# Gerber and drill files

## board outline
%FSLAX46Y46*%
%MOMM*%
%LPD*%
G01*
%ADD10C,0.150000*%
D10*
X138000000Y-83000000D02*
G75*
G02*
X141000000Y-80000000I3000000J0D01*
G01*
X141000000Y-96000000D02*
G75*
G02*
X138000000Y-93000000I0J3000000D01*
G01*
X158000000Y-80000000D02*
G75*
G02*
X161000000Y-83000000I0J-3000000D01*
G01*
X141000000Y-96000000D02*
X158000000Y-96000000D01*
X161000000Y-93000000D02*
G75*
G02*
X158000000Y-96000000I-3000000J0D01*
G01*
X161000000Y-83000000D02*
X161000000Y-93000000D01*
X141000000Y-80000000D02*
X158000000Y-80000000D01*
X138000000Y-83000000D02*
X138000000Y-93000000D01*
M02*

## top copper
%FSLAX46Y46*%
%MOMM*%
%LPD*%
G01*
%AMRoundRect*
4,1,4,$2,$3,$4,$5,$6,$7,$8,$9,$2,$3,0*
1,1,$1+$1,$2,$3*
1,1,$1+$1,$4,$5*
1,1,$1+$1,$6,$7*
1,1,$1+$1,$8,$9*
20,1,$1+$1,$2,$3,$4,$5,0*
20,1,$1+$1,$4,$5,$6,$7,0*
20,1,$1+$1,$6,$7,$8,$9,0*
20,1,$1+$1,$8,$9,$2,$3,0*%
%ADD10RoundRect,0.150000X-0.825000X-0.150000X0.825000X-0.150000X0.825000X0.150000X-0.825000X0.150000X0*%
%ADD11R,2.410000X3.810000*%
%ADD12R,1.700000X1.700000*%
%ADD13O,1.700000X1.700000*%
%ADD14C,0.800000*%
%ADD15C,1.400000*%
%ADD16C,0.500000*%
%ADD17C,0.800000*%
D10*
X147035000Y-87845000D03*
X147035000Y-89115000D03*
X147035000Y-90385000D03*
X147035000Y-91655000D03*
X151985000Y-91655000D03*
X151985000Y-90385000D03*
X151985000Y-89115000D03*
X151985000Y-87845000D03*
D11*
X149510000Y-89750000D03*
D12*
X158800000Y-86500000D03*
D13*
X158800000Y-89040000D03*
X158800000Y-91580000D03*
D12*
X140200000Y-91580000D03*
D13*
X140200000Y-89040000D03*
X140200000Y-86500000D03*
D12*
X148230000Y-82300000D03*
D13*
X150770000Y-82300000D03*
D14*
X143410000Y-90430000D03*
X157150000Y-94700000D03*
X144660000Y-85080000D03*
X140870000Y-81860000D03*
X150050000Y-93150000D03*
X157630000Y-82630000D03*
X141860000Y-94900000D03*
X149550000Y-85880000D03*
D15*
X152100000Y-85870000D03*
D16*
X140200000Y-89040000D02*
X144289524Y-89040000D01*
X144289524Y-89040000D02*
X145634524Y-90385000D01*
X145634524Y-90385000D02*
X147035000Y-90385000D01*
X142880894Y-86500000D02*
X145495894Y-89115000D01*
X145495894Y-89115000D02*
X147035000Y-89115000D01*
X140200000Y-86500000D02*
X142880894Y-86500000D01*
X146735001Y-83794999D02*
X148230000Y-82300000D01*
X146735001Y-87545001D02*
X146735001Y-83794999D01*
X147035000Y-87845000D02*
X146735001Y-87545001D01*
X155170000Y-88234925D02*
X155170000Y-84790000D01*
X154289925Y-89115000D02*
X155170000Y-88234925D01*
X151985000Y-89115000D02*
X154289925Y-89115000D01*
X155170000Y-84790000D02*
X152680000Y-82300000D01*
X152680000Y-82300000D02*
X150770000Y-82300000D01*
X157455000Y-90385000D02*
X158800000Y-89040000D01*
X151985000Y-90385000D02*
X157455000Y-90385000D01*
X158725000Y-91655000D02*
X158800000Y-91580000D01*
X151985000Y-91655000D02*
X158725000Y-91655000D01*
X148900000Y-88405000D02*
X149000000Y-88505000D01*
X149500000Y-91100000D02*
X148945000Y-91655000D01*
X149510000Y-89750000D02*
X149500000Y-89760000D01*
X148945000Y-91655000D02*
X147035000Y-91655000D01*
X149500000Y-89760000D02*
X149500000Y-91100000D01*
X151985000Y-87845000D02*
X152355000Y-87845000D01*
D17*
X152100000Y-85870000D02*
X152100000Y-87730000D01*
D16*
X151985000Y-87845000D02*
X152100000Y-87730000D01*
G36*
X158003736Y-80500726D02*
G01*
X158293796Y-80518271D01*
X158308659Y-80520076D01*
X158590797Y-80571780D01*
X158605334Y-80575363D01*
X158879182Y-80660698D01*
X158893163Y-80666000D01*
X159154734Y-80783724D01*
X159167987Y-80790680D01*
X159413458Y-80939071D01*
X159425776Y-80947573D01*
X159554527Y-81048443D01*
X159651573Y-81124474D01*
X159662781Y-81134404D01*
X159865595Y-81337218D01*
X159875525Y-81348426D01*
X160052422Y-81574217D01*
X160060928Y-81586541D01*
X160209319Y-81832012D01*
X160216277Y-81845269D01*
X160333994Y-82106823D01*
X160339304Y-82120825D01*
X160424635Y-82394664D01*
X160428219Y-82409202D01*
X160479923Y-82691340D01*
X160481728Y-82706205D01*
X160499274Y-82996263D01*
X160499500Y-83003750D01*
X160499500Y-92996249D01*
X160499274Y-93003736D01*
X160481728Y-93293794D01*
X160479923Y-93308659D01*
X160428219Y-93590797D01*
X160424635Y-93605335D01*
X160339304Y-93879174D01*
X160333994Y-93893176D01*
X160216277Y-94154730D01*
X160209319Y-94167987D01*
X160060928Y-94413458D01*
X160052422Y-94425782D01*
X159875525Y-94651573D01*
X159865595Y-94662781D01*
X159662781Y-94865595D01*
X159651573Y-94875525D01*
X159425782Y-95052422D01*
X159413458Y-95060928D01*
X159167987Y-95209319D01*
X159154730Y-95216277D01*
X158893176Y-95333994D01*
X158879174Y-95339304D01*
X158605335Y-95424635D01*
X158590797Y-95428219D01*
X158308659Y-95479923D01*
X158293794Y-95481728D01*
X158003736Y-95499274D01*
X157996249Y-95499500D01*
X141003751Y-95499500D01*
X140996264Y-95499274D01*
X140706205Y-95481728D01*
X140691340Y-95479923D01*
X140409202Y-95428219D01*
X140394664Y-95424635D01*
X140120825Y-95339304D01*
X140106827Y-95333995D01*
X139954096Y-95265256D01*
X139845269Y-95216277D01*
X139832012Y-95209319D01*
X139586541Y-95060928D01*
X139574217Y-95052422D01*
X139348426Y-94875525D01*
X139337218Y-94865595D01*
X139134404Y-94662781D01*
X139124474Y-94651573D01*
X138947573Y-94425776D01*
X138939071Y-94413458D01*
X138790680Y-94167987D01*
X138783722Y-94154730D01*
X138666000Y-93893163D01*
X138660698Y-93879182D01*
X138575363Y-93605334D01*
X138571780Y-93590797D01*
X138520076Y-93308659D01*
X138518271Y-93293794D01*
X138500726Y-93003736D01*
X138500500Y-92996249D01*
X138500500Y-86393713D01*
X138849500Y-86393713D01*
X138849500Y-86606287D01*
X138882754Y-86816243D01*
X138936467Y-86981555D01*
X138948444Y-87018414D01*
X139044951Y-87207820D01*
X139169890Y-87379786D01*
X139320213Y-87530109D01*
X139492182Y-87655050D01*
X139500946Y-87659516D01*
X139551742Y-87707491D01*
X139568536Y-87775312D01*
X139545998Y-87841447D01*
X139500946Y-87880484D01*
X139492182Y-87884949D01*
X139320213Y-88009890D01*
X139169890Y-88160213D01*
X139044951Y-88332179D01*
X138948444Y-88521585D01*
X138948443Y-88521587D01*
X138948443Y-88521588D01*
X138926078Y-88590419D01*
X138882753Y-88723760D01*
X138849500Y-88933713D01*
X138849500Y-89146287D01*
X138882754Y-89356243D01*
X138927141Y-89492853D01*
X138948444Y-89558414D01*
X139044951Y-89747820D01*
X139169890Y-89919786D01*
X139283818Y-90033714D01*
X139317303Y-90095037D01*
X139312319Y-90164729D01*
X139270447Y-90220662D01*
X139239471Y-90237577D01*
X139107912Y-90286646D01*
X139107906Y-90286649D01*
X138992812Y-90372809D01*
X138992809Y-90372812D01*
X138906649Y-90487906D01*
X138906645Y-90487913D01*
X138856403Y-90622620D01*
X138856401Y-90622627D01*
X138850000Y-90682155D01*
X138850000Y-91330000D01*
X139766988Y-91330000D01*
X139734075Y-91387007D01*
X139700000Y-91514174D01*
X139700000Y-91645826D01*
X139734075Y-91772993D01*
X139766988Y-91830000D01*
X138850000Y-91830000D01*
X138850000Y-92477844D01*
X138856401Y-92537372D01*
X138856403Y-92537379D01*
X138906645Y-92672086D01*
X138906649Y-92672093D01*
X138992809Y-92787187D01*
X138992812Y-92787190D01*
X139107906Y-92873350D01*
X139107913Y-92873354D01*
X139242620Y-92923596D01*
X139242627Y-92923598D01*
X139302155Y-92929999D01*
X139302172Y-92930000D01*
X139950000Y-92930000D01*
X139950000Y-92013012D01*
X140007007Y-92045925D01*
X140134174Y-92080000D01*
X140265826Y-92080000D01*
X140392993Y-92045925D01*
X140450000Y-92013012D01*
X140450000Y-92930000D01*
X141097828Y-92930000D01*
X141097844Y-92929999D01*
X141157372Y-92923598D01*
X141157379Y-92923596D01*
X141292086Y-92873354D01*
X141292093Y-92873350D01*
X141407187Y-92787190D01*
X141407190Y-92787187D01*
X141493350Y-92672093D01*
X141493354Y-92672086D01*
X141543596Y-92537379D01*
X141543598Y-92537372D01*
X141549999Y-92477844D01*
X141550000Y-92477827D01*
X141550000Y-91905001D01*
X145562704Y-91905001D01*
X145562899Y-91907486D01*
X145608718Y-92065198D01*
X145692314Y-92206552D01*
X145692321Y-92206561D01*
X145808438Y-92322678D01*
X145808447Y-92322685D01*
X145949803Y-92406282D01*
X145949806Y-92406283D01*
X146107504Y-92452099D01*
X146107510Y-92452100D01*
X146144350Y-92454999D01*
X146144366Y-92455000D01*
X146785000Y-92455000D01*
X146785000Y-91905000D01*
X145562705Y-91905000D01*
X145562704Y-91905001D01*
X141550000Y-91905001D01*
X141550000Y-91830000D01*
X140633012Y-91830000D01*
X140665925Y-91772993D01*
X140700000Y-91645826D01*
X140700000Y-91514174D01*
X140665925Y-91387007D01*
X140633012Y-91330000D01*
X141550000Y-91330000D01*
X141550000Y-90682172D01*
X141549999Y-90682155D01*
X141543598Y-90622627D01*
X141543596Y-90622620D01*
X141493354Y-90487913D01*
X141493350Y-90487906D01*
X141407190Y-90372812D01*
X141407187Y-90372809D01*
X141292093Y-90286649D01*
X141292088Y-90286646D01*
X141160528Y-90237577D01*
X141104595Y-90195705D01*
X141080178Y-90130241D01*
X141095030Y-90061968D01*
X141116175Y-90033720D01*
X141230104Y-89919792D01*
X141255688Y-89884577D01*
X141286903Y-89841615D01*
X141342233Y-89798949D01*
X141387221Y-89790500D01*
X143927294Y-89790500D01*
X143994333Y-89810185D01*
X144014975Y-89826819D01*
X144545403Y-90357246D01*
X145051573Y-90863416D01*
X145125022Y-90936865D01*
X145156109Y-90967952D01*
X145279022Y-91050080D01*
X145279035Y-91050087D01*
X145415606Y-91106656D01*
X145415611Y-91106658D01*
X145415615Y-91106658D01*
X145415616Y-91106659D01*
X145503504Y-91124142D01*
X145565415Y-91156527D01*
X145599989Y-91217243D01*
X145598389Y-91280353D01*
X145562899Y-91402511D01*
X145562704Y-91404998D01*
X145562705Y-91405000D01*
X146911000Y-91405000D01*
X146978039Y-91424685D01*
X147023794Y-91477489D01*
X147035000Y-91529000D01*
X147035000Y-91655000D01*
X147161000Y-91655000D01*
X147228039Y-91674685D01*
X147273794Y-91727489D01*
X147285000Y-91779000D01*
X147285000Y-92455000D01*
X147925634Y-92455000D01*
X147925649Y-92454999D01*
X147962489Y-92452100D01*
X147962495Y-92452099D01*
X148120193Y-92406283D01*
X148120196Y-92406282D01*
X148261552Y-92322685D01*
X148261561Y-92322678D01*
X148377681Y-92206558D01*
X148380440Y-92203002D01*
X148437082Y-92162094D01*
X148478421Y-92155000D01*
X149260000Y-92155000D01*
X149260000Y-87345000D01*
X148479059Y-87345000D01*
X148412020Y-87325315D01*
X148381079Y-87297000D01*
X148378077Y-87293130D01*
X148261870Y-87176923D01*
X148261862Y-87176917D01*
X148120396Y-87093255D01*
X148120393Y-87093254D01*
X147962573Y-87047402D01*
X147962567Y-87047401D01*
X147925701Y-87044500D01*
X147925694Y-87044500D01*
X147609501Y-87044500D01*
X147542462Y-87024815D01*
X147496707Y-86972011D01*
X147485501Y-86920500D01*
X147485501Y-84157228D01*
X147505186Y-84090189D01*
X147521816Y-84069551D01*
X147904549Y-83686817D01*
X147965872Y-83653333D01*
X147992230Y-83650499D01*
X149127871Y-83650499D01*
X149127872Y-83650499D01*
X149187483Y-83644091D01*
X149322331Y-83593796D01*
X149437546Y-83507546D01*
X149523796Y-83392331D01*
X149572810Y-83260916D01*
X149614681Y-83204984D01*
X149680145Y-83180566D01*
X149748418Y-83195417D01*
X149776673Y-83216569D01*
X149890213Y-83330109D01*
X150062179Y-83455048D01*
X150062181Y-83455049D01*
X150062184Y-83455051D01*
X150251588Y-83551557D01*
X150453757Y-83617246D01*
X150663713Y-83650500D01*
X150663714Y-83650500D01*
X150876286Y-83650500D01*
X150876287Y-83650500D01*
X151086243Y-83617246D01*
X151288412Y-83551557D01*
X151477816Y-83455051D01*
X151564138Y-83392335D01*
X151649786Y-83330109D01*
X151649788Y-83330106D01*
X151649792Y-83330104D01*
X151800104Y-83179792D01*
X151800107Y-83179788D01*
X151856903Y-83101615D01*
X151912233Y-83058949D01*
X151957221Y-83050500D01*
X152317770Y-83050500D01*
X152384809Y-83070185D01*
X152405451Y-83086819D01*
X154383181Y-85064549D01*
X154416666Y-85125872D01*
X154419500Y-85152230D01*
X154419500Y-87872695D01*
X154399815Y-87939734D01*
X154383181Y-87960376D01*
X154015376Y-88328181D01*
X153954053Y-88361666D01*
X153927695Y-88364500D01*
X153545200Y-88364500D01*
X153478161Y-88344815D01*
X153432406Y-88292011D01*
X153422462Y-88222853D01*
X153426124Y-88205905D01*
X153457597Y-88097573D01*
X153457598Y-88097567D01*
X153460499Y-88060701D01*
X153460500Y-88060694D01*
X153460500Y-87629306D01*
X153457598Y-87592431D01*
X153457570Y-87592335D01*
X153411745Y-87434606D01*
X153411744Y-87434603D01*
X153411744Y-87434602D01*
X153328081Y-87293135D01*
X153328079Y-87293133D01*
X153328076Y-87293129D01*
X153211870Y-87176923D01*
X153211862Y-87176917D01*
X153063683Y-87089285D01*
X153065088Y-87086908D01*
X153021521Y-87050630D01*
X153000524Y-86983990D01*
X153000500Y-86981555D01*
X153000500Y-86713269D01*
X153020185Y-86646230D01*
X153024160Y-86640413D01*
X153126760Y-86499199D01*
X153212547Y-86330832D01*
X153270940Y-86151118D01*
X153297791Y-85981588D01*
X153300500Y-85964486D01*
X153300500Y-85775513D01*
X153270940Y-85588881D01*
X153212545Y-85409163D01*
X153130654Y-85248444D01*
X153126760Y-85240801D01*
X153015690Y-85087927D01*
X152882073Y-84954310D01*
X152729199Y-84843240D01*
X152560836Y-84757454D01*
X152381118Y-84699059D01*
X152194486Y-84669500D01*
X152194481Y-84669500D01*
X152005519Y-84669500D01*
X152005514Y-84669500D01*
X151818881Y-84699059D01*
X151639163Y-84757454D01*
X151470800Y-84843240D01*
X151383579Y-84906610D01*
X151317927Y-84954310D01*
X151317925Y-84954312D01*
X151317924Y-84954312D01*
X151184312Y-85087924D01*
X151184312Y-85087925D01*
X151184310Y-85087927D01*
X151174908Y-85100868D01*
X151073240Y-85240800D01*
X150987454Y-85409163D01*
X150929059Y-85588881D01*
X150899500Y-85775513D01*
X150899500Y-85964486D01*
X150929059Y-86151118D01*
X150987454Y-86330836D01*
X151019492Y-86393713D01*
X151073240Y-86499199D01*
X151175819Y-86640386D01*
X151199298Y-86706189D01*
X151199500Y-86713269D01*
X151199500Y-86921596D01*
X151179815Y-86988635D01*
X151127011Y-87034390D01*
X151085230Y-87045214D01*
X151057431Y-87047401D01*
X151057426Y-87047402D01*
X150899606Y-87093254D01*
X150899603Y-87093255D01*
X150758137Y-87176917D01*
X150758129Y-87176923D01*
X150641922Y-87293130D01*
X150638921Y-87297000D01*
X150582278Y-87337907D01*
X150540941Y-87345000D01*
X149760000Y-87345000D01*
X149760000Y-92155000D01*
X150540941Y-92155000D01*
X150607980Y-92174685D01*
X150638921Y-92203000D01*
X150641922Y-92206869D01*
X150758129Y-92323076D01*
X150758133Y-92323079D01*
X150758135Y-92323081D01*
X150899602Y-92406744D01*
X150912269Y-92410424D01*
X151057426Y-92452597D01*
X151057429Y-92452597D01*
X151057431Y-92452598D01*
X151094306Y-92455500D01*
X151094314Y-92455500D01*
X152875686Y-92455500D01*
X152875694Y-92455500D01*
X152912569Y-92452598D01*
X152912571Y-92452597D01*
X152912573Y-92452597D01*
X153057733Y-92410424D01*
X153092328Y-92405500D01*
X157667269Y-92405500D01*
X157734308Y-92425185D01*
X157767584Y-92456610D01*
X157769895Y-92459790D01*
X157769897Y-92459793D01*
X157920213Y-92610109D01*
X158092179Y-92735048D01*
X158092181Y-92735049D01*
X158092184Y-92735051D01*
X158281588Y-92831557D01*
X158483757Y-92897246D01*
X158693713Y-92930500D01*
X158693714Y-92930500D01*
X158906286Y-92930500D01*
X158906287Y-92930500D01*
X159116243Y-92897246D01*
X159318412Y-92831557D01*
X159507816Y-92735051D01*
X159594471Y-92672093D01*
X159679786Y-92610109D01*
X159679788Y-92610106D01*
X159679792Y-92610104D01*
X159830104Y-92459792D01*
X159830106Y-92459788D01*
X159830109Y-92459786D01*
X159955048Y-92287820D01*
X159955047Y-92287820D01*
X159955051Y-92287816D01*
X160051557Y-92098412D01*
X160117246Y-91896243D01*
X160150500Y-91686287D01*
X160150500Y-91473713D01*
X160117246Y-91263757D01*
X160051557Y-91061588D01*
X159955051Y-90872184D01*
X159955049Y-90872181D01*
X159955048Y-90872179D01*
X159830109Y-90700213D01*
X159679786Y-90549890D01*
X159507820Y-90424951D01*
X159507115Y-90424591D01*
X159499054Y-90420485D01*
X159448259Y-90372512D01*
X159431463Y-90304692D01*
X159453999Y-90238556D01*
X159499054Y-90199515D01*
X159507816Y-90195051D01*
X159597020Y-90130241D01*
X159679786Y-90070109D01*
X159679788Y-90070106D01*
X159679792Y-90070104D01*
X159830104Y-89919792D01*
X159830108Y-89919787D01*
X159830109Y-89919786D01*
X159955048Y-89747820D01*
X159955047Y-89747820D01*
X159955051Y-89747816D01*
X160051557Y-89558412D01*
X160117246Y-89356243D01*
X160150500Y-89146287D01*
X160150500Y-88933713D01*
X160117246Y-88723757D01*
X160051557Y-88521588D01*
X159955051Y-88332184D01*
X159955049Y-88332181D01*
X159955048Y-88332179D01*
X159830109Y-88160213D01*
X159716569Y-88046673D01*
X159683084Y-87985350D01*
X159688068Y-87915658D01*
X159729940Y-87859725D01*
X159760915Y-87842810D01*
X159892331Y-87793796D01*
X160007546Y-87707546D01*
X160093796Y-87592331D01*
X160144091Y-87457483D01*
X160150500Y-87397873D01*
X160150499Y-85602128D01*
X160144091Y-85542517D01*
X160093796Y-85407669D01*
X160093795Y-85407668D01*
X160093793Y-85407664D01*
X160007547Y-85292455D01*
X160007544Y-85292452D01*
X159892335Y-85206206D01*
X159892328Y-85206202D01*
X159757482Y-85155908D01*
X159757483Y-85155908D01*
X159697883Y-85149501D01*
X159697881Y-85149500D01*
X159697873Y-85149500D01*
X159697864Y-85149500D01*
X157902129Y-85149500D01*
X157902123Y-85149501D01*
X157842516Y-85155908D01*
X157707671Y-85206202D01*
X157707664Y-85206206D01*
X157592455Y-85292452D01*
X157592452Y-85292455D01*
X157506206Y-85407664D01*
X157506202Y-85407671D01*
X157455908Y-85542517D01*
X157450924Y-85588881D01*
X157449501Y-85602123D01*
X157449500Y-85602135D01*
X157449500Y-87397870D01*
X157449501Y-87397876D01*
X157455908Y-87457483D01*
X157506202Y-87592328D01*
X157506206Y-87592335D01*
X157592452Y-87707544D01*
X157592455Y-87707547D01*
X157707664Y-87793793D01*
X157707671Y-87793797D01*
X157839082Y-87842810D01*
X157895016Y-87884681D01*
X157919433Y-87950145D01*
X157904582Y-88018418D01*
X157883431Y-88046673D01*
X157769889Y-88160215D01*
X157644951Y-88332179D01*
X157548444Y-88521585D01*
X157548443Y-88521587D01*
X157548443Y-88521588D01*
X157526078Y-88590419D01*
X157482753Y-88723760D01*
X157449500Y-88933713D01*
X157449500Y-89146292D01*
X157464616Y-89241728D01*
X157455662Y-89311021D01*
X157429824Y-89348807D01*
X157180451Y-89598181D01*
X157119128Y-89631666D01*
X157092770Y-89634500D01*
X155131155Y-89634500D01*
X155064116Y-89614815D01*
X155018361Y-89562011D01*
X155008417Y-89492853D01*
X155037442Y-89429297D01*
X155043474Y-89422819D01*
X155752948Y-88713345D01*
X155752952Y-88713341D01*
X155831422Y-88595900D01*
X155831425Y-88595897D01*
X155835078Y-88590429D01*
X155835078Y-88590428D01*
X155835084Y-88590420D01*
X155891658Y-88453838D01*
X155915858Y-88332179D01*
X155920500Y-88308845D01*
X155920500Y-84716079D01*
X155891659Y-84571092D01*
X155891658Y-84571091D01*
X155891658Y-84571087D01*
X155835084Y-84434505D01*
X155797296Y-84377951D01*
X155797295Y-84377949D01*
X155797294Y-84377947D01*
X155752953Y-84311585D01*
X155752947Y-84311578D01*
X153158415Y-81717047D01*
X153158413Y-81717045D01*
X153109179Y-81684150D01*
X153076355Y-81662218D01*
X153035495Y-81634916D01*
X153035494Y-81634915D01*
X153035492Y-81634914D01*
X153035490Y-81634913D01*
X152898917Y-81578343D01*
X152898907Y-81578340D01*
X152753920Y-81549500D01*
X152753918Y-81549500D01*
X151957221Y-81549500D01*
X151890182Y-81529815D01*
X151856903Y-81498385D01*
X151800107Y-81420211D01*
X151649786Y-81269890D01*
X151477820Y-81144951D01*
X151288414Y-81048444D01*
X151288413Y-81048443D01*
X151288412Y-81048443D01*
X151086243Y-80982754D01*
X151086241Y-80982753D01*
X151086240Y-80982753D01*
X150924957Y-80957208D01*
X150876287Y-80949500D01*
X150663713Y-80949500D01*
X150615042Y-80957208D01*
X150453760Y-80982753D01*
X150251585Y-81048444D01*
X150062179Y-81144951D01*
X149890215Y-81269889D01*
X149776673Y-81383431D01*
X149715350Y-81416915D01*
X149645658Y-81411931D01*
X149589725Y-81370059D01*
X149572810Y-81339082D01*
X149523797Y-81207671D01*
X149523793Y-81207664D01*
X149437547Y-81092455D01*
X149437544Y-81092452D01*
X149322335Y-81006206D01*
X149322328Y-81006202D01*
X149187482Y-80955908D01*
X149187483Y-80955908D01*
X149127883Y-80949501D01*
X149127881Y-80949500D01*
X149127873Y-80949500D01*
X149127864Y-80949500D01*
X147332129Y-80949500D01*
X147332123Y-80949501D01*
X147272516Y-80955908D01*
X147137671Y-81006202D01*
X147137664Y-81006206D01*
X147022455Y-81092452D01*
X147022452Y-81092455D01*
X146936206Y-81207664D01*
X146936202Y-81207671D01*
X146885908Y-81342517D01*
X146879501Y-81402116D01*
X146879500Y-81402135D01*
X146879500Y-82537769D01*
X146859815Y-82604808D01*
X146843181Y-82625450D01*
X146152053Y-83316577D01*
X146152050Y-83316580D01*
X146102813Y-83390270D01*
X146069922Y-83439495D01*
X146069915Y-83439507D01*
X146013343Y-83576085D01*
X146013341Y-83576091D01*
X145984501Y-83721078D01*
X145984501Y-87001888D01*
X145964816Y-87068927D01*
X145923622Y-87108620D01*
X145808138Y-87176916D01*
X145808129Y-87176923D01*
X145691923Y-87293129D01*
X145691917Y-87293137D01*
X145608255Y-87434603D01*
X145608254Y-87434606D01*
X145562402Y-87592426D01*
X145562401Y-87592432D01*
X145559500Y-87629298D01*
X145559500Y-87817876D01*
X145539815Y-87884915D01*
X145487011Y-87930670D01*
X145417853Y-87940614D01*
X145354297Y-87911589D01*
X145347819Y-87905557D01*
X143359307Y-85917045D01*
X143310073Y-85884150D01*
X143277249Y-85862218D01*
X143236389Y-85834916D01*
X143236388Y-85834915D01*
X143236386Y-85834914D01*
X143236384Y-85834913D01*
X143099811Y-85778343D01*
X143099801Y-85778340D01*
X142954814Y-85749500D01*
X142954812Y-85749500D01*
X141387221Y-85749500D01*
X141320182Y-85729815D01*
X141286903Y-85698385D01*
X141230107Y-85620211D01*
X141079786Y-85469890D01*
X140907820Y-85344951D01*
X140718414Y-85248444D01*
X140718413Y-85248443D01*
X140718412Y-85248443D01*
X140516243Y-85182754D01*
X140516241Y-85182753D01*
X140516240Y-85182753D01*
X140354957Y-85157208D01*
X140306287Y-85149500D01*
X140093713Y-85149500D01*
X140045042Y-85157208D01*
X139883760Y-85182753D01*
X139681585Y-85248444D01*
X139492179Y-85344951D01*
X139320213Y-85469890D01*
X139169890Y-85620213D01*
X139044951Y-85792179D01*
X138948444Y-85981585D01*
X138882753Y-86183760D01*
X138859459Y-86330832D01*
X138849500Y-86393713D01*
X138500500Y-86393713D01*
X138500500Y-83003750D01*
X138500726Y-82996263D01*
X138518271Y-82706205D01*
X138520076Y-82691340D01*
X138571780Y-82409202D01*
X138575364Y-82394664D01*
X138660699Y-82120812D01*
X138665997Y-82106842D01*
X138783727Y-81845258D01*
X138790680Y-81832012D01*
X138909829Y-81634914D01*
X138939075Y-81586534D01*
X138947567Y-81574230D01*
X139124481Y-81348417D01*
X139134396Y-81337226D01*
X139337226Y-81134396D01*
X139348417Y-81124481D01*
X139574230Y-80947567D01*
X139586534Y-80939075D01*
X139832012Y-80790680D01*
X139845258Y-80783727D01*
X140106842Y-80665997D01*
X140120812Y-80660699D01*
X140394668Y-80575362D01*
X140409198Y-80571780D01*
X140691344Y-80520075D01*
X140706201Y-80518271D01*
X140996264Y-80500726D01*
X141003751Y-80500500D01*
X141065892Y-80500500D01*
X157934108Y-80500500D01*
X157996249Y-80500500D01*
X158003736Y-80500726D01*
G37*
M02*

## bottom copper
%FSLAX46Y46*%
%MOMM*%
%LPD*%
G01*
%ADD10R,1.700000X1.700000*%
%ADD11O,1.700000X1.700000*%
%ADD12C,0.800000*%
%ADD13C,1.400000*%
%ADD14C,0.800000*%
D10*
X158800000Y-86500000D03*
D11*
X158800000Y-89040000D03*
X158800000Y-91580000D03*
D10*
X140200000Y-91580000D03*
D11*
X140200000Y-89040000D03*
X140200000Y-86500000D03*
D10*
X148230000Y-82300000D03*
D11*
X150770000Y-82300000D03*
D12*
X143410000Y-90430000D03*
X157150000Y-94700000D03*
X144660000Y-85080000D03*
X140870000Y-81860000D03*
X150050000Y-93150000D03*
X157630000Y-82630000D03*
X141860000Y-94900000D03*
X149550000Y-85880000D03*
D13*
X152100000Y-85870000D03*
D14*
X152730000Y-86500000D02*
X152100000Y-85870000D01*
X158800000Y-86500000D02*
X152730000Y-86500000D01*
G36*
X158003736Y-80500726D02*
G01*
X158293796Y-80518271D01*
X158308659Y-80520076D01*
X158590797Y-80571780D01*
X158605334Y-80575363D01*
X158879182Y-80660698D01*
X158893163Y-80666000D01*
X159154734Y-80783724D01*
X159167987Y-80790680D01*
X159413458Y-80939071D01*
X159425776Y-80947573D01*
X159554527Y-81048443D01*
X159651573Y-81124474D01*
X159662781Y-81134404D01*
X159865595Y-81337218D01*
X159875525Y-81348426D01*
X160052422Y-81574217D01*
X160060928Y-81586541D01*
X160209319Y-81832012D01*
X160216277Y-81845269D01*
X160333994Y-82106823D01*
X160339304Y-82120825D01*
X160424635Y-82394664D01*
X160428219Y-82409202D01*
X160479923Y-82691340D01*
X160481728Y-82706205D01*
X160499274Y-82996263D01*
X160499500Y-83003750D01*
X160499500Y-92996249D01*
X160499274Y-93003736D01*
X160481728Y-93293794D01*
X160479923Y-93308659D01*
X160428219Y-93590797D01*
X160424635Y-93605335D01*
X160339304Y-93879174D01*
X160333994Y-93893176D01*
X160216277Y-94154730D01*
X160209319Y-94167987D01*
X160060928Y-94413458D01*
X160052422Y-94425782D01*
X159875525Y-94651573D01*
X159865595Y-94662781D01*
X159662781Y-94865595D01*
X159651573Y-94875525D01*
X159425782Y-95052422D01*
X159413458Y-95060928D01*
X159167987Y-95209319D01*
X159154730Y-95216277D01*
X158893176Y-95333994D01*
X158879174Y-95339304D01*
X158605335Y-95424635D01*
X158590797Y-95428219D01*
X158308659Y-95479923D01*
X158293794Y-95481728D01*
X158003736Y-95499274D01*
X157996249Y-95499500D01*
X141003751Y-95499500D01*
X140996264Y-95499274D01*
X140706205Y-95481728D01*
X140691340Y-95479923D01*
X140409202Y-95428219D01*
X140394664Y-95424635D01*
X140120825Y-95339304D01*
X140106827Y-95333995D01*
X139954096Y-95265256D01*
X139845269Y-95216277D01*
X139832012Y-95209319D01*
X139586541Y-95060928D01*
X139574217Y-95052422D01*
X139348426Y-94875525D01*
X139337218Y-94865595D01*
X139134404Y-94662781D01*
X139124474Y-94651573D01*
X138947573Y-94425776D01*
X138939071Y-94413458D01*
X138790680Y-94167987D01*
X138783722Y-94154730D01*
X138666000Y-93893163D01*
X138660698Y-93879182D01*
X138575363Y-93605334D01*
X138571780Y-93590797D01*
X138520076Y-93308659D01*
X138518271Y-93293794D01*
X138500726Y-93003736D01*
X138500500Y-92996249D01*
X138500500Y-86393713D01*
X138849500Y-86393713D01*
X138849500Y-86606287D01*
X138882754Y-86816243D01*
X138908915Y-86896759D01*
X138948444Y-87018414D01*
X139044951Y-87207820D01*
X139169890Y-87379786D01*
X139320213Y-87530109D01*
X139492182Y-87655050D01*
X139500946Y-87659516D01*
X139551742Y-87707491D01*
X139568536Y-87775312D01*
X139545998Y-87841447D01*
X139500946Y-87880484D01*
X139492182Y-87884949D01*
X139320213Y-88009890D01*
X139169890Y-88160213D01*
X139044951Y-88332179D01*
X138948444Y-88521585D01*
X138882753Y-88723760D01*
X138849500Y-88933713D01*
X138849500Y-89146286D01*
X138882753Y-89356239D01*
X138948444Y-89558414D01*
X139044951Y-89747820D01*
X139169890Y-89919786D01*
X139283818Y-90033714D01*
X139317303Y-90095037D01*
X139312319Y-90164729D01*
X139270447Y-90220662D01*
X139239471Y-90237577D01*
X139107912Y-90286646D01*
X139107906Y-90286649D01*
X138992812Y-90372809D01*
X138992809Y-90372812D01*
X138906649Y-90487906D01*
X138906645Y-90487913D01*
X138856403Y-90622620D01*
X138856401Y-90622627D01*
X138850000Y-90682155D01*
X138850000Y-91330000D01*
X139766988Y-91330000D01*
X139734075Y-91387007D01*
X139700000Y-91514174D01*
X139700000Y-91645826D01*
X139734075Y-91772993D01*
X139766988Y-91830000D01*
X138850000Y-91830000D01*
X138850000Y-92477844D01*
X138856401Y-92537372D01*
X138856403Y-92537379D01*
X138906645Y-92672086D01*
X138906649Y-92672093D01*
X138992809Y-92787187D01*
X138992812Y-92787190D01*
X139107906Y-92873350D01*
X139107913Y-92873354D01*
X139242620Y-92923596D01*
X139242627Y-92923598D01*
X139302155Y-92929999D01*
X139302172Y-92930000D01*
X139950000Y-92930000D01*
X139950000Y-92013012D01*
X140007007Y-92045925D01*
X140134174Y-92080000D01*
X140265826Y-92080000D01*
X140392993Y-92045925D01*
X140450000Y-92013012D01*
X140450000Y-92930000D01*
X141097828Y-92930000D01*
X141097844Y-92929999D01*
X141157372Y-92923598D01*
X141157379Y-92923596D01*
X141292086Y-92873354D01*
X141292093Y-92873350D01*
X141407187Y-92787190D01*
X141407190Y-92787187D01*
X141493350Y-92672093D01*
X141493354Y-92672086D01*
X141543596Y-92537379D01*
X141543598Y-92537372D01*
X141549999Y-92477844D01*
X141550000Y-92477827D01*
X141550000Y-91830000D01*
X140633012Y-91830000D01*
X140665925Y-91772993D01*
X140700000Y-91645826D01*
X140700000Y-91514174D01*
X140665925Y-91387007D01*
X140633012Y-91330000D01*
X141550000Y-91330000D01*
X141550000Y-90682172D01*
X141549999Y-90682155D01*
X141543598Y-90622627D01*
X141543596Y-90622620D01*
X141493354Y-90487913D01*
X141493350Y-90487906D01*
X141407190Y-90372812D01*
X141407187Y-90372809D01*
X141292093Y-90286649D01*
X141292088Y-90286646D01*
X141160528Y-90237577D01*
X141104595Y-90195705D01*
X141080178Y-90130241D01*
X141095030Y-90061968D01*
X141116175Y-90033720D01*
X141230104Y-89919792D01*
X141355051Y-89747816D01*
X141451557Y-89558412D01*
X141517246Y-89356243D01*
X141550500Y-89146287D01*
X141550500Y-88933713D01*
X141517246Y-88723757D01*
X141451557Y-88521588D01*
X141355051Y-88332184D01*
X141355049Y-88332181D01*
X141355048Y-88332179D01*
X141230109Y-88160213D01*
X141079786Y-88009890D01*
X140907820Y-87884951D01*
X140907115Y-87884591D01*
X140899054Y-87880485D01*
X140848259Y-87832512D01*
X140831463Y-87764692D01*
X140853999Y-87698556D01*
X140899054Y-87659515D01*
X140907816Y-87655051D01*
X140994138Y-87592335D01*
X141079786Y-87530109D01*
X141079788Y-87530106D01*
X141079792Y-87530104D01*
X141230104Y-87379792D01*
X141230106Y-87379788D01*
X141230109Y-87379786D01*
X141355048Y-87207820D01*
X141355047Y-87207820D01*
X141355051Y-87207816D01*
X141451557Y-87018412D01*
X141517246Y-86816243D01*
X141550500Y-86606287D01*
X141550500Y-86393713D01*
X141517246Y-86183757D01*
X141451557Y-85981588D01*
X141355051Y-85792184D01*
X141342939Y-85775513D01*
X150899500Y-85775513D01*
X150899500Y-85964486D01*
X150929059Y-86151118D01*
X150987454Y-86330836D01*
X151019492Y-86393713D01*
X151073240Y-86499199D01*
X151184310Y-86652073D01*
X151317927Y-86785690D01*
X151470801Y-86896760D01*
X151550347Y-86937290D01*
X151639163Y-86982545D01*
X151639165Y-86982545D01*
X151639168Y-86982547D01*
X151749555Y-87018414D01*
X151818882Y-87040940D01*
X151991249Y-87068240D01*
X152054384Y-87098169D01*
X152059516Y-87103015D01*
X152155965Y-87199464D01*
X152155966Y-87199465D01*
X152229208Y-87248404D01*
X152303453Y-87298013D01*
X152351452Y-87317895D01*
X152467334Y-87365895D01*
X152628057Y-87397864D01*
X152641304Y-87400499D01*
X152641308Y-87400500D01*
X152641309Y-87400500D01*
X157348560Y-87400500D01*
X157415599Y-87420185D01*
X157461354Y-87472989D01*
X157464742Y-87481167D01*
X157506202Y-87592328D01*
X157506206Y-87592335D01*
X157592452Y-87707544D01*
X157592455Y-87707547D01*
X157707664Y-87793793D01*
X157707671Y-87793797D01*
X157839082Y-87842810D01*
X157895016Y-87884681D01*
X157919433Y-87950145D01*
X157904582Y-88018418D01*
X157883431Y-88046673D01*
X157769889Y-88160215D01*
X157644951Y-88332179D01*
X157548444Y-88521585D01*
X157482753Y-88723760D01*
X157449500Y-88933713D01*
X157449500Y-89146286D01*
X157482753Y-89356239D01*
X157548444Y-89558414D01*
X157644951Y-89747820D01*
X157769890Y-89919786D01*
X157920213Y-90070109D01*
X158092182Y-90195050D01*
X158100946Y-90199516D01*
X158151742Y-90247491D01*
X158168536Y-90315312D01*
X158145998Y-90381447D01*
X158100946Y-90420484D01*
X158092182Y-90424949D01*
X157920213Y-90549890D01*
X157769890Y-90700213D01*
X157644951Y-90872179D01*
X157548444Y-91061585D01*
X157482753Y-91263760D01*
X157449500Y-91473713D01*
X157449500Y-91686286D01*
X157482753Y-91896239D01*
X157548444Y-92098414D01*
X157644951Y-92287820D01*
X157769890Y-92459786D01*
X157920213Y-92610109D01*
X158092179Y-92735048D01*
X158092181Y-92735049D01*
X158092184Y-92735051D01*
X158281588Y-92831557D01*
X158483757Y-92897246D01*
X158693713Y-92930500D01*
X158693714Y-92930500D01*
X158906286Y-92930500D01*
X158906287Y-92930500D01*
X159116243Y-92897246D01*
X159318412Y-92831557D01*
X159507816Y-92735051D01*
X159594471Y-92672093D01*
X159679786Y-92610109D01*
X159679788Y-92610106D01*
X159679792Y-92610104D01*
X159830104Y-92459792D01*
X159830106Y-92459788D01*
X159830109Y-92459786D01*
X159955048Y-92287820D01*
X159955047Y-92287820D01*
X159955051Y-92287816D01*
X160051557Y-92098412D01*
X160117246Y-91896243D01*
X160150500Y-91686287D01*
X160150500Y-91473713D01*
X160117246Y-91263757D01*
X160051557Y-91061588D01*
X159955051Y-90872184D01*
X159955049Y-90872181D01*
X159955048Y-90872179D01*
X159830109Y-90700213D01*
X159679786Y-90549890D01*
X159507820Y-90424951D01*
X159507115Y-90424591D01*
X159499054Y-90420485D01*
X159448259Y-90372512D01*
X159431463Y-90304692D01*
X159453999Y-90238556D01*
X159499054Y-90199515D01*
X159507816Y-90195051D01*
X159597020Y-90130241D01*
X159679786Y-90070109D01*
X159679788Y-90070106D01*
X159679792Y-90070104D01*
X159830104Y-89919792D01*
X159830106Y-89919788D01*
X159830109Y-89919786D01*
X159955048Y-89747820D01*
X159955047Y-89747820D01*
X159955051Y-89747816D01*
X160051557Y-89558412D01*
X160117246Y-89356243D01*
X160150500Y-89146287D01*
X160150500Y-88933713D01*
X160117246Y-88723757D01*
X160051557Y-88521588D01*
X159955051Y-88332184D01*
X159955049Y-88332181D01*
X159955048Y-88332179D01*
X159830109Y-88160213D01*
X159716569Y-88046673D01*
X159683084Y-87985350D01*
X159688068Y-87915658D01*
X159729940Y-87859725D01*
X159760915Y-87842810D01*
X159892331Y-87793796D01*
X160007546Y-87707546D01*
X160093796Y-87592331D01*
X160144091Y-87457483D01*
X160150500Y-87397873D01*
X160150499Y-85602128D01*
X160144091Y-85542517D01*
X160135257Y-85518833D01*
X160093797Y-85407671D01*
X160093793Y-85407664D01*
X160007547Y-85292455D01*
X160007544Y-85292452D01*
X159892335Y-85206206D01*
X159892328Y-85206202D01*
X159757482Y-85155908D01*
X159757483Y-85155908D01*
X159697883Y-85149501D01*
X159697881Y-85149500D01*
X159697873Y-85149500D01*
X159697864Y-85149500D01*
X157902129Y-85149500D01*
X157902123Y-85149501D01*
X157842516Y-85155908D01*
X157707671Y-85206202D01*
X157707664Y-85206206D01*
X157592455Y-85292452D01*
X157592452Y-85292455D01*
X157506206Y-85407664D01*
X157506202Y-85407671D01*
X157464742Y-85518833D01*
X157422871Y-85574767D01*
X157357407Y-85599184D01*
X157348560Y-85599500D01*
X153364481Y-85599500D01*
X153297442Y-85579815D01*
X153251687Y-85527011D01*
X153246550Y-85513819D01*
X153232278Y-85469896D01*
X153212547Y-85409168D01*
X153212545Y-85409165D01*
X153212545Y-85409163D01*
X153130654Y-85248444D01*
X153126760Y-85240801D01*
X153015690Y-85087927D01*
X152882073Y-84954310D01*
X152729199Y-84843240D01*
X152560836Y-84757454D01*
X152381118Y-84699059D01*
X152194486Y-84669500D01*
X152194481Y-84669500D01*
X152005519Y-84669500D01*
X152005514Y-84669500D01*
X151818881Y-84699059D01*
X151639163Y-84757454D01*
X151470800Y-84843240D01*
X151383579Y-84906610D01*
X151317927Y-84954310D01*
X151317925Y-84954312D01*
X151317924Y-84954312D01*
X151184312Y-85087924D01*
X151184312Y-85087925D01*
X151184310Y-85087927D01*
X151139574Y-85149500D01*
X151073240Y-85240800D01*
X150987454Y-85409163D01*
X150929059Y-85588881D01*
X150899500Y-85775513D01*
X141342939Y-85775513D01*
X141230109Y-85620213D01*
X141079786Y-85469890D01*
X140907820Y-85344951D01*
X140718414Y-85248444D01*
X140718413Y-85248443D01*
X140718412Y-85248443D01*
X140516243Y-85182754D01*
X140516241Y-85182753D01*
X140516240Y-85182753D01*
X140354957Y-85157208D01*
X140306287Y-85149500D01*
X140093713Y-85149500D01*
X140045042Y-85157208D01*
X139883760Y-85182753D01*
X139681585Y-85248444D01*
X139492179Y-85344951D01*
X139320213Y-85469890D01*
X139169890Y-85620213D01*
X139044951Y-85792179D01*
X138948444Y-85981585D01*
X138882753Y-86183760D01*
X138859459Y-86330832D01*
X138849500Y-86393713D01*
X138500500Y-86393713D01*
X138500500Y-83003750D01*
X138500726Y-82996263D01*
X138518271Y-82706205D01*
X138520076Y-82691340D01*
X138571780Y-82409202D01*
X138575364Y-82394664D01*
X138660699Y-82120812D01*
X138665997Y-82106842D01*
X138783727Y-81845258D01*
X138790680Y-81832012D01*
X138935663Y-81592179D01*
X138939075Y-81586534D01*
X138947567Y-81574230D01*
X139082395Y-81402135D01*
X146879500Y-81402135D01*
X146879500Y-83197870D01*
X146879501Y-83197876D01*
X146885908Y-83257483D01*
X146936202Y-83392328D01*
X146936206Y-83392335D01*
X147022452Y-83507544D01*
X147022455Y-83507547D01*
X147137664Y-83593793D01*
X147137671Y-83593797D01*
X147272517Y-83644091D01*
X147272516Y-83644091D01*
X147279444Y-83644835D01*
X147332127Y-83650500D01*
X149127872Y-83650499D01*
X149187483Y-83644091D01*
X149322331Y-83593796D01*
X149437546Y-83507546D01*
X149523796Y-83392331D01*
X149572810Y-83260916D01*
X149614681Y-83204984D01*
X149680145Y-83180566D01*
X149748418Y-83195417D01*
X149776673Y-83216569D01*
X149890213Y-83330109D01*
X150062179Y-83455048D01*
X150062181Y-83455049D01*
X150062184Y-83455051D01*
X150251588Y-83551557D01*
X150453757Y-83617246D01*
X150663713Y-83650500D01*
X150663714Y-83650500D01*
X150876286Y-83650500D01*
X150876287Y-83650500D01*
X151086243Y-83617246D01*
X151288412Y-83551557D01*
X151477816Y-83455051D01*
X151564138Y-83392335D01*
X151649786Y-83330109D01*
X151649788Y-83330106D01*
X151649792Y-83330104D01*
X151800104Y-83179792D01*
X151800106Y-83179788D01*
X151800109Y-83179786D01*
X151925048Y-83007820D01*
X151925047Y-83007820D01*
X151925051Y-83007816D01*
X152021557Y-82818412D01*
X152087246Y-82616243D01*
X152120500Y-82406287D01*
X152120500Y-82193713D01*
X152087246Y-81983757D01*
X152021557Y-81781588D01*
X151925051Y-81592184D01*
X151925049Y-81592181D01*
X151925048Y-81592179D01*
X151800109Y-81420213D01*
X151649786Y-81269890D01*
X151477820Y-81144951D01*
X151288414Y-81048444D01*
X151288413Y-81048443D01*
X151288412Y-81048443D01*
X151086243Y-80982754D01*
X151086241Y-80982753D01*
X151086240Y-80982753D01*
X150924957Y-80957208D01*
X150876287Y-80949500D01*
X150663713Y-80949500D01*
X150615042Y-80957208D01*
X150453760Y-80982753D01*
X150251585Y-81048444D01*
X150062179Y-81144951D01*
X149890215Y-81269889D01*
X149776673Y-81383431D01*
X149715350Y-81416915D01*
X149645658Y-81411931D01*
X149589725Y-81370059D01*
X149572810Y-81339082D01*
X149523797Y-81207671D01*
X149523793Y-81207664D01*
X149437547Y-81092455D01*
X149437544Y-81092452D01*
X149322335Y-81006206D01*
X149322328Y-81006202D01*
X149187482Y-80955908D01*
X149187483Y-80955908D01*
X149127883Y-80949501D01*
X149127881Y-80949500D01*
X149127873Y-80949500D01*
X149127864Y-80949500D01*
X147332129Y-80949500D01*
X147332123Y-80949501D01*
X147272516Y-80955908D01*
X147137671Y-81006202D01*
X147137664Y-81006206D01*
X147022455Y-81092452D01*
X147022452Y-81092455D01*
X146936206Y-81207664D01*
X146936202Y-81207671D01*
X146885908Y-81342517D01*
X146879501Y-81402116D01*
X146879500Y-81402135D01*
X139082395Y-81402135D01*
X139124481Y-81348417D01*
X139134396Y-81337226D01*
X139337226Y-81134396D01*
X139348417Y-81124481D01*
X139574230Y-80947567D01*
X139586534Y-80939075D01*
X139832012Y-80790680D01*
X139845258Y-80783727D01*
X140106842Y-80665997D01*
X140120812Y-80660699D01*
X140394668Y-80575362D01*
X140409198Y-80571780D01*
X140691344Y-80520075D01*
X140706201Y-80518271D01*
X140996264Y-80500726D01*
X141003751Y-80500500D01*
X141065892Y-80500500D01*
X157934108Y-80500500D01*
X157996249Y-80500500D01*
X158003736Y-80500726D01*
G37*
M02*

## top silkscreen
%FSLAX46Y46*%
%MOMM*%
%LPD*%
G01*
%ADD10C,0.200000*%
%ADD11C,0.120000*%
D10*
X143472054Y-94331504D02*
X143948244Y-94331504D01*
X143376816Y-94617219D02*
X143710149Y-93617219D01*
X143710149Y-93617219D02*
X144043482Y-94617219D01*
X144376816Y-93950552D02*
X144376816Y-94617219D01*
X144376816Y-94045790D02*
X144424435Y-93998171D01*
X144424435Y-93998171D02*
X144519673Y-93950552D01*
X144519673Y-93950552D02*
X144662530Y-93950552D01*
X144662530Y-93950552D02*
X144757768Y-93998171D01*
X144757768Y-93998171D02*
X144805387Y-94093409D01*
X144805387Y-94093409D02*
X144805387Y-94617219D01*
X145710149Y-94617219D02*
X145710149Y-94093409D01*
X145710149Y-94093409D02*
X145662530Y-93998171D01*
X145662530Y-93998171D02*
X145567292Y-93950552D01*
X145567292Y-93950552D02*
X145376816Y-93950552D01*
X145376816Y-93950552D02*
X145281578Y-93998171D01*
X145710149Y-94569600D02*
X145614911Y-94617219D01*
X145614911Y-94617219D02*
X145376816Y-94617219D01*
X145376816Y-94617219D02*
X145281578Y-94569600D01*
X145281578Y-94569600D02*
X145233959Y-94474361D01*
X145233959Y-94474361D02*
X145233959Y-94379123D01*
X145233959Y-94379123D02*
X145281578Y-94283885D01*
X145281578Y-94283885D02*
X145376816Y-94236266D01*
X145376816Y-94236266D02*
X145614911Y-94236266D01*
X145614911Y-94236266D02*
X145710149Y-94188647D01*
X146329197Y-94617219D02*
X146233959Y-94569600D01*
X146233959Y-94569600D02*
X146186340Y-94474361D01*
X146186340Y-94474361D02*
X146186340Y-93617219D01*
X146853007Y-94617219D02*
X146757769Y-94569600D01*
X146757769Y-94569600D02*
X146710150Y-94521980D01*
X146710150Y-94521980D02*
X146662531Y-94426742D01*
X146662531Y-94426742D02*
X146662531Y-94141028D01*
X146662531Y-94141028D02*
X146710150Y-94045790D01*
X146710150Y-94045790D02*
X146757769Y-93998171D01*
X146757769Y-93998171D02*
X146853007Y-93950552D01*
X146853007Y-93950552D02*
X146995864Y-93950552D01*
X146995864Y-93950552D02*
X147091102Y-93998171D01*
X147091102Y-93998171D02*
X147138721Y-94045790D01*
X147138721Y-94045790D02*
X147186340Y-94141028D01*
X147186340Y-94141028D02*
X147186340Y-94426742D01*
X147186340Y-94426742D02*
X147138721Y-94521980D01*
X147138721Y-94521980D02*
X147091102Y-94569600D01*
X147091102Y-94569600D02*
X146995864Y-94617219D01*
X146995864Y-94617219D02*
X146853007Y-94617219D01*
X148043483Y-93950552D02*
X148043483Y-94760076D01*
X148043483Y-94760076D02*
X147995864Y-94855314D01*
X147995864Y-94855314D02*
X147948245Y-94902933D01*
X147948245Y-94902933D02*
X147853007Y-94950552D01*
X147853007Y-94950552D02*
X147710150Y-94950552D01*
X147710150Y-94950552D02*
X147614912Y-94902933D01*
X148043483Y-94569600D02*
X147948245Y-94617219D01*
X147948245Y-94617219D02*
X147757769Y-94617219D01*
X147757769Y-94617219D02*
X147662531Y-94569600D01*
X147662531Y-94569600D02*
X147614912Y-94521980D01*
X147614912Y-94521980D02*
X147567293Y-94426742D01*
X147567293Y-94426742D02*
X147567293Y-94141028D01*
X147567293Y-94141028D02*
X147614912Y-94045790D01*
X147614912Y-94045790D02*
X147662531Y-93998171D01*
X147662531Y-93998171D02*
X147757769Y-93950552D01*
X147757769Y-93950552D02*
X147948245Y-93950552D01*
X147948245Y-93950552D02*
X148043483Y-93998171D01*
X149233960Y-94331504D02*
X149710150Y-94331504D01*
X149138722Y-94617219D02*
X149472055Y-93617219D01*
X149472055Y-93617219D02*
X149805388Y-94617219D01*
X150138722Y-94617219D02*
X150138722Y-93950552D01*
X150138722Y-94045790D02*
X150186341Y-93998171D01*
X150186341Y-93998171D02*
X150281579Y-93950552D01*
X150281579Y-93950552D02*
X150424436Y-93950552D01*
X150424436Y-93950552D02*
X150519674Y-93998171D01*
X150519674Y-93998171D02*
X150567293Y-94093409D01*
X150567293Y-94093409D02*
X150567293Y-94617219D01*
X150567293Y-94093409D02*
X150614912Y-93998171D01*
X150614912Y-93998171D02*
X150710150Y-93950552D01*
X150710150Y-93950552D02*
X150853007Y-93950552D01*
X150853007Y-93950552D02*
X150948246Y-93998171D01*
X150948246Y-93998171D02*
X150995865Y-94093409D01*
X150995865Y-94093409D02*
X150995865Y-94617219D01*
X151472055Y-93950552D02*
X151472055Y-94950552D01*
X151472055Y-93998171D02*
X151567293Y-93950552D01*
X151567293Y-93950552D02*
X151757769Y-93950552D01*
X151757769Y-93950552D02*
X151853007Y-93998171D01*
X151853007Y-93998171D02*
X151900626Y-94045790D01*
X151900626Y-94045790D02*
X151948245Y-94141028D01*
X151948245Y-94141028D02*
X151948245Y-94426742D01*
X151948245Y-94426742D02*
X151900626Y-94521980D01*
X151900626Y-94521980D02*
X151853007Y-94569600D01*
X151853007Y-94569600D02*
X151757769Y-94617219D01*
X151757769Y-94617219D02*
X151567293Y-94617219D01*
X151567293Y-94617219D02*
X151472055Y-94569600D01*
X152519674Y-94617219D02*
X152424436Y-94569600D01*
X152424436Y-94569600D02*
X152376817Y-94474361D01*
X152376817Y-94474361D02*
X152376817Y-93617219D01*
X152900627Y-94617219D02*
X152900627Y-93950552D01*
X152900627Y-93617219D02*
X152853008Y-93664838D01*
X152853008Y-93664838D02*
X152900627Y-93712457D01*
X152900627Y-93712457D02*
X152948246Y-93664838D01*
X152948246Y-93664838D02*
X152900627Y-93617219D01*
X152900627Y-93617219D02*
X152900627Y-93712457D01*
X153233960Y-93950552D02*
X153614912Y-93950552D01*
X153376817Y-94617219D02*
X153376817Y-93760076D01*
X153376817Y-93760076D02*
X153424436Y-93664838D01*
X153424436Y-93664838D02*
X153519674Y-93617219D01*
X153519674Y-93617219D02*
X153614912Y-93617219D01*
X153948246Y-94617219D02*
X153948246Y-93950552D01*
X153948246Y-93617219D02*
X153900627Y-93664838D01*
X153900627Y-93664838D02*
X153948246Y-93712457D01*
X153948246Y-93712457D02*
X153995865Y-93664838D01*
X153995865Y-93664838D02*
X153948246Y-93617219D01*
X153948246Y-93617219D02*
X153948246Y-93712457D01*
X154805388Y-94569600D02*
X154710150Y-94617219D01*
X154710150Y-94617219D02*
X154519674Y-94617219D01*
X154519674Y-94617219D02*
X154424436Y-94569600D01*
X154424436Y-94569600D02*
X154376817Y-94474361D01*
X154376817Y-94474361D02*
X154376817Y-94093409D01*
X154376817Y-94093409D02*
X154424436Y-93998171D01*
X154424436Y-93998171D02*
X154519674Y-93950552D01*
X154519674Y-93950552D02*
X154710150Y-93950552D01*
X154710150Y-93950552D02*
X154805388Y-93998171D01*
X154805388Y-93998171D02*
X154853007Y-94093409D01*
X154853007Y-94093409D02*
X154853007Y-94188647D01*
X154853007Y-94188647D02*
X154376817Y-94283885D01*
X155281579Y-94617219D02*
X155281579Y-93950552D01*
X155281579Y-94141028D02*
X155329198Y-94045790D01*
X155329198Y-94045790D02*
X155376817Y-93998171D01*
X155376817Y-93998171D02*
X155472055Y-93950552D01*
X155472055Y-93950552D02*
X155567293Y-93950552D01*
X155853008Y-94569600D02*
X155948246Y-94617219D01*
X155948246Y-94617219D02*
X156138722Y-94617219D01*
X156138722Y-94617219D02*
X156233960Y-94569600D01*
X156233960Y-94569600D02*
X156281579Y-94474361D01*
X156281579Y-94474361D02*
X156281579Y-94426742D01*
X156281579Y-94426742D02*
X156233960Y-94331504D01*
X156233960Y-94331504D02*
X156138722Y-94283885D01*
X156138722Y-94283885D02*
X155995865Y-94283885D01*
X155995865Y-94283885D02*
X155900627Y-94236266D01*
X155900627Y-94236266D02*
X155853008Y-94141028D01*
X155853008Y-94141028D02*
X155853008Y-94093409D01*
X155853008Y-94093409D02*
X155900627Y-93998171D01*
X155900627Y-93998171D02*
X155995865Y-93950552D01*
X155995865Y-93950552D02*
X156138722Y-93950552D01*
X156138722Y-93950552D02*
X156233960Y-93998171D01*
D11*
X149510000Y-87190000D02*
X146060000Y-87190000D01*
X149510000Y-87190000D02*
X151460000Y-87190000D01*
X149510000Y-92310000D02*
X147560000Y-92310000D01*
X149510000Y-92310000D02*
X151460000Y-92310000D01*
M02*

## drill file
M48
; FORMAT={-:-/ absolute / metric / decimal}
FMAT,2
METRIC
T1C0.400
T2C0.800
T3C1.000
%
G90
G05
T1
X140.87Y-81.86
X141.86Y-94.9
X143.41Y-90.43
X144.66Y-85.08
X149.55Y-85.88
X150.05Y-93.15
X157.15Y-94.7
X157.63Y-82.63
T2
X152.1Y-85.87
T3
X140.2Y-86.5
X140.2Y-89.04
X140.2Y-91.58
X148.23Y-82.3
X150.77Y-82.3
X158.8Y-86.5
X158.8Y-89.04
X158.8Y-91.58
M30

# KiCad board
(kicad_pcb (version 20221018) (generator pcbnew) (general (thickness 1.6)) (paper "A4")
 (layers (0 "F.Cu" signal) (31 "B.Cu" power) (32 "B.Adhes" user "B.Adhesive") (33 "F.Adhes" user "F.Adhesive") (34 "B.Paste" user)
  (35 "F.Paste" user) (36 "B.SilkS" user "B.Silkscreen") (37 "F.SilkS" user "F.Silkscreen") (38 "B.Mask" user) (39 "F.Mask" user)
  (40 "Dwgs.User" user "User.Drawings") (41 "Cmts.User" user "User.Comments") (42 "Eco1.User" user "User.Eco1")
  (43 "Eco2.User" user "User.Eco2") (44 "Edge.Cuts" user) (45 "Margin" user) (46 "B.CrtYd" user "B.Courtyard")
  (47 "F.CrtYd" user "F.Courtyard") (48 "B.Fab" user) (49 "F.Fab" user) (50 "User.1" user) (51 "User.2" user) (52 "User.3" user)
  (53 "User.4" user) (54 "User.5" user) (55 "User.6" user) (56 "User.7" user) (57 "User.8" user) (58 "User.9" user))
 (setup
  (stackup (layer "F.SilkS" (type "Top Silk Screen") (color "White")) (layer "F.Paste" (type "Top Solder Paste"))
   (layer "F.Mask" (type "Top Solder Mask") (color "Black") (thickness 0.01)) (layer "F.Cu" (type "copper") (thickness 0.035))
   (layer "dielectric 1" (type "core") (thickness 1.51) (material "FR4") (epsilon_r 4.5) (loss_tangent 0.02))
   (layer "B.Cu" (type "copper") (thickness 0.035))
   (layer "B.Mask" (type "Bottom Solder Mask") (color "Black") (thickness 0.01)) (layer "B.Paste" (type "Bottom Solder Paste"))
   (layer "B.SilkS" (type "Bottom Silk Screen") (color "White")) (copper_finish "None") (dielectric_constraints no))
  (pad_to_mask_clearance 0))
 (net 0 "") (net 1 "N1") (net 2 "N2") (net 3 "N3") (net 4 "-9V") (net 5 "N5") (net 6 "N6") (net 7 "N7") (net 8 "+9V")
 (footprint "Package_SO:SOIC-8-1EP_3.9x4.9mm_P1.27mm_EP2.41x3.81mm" (layer "F.Cu") (at 149.51 89.75)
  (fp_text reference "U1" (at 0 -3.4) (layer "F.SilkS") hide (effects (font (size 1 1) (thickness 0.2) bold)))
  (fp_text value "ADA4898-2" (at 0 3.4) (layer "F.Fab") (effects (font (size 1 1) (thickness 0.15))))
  (fp_line (start 0 -2.56) (end -3.45 -2.56) (stroke (width 0.12) (type solid)) (layer "F.SilkS"))
  (fp_line (start 0 -2.56) (end 1.95 -2.56) (stroke (width 0.12) (type solid)) (layer "F.SilkS"))
  (fp_line (start 0 2.56) (end -1.95 2.56) (stroke (width 0.12) (type solid)) (layer "F.SilkS"))
  (fp_line (start 0 2.56) (end 1.95 2.56) (stroke (width 0.12) (type solid)) (layer "F.SilkS"))
  (pad "" smd roundrect (at -0.6 -0.95) (size 0.97 1.54) (layers "F.Paste") (roundrect_rratio 0.25))
  (pad "" smd roundrect (at -0.6 0.95) (size 0.97 1.54) (layers "F.Paste") (roundrect_rratio 0.25))
  (pad "" smd roundrect (at 0.6 -0.95) (size 0.97 1.54) (layers "F.Paste") (roundrect_rratio 0.25))
  (pad "" smd roundrect (at 0.6 0.95) (size 0.97 1.54) (layers "F.Paste") (roundrect_rratio 0.25))
  (pad "1" smd roundrect (at -2.475 -1.905) (size 1.95 0.6) (layers "F.Cu" "F.Paste" "F.Mask") (roundrect_rratio 0.25) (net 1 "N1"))
  (pad "2" smd roundrect (at -2.475 -0.635) (size 1.95 0.6) (layers "F.Cu" "F.Paste" "F.Mask") (roundrect_rratio 0.25) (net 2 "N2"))
  (pad "3" smd roundrect (at -2.475 0.635) (size 1.95 0.6) (layers "F.Cu" "F.Paste" "F.Mask") (roundrect_rratio 0.25) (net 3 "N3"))
  (pad "4" smd roundrect (at -2.475 1.905) (size 1.95 0.6) (layers "F.Cu" "F.Paste" "F.Mask") (roundrect_rratio 0.25) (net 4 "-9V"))
  (pad "5" smd roundrect (at 2.475 1.905) (size 1.95 0.6) (layers "F.Cu" "F.Paste" "F.Mask") (roundrect_rratio 0.25) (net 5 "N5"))
  (pad "6" smd roundrect (at 2.475 0.635) (size 1.95 0.6) (layers "F.Cu" "F.Paste" "F.Mask") (roundrect_rratio 0.25) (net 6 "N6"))
  (pad "7" smd roundrect (at 2.475 -0.635) (size 1.95 0.6) (layers "F.Cu" "F.Paste" "F.Mask") (roundrect_rratio 0.25) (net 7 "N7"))
  (pad "8" smd roundrect (at 2.475 -1.905) (size 1.95 0.6) (layers "F.Cu" "F.Paste" "F.Mask") (roundrect_rratio 0.25) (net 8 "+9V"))
  (pad "9" smd rect (at 0 0) (size 2.41 3.81) (layers "F.Cu" "F.Mask") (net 4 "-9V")))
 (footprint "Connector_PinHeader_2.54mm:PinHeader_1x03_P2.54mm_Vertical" (layer "B.Cu") (at 158.8 86.5 180)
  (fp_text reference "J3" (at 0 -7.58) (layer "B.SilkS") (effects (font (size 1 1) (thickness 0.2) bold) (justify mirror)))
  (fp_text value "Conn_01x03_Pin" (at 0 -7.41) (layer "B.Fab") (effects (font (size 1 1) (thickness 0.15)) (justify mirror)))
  (pad "1" thru_hole rect (at 0 0 180) (size 1.7 1.7) (drill 1) (layers "*.Cu" "*.Mask") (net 8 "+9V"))
  (pad "2" thru_hole oval (at 0 -2.54 180) (size 1.7 1.7) (drill 1) (layers "*.Cu" "*.Mask") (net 6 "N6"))
  (pad "3" thru_hole oval (at 0 -5.08 180) (size 1.7 1.7) (drill 1) (layers "*.Cu" "*.Mask") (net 5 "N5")))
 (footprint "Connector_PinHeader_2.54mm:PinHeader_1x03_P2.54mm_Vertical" (layer "B.Cu") (at 140.2 91.58)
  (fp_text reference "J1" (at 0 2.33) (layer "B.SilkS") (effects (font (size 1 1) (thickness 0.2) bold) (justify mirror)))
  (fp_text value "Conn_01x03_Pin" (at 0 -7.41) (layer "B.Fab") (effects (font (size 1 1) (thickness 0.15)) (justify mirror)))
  (pad "1" thru_hole rect (at 0 0) (size 1.7 1.7) (drill 1) (layers "*.Cu" "*.Mask") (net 4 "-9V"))
  (pad "2" thru_hole oval (at 0 -2.54) (size 1.7 1.7) (drill 1) (layers "*.Cu" "*.Mask") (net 3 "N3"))
  (pad "3" thru_hole oval (at 0 -5.08) (size 1.7 1.7) (drill 1) (layers "*.Cu" "*.Mask") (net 2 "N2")))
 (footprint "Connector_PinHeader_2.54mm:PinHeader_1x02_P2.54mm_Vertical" (layer "B.Cu") (at 148.23 82.3 -90)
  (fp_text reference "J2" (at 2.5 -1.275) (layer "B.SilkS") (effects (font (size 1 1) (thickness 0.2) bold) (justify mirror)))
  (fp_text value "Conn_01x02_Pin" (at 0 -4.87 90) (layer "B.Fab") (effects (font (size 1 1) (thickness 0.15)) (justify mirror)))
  (pad "1" thru_hole rect (at 0 0 270) (size 1.7 1.7) (drill 1) (layers "*.Cu" "*.Mask") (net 1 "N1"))
  (pad "2" thru_hole oval (at 0 -2.54 270) (size 1.7 1.7) (drill 1) (layers "*.Cu" "*.Mask") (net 7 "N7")))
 (gr_arc (start 138 83) (mid 138.87868 80.87868) (end 141 80) (stroke (width 0.15) (type default)) (layer "Edge.Cuts"))
 (gr_arc (start 141 96) (mid 138.87868 95.12132) (end 138 93) (stroke (width 0.15) (type default)) (layer "Edge.Cuts"))
 (gr_arc (start 158 80) (mid 160.12132 80.87868) (end 161 83) (stroke (width 0.15) (type default)) (layer "Edge.Cuts"))
 (gr_line (start 141 96) (end 158 96) (stroke (width 0.15) (type default)) (layer "Edge.Cuts"))
 (gr_arc (start 161 93) (mid 160.12132 95.12132) (end 158 96) (stroke (width 0.15) (type default)) (layer "Edge.Cuts"))
 (gr_line (start 161 83) (end 161 93) (stroke (width 0.15) (type default)) (layer "Edge.Cuts"))
 (gr_line (start 141 80) (end 158 80) (stroke (width 0.15) (type default)) (layer "Edge.Cuts"))
 (gr_line (start 138 83) (end 138 93) (stroke (width 0.15) (type default)) (layer "Edge.Cuts"))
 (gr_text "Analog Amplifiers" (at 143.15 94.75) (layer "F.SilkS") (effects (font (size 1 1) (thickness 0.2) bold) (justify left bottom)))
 (segment (start 140.2 89.04) (end 144.289524 89.04) (width 0.5) (layer "F.Cu") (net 3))
 (segment (start 144.289524 89.04) (end 145.634524 90.385) (width 0.5) (layer "F.Cu") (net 3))
 (segment (start 145.634524 90.385) (end 147.035 90.385) (width 0.5) (layer "F.Cu") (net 3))
 (segment (start 142.880894 86.5) (end 145.495894 89.115) (width 0.5) (layer "F.Cu") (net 2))
 (segment (start 145.495894 89.115) (end 147.035 89.115) (width 0.5) (layer "F.Cu") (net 2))
 (segment (start 140.2 86.5) (end 142.880894 86.5) (width 0.5) (layer "F.Cu") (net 2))
 (segment (start 146.735001 83.794999) (end 148.23 82.3) (width 0.5) (layer "F.Cu") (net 1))
 (segment (start 146.735001 87.545001) (end 146.735001 83.794999) (width 0.5) (layer "F.Cu") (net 1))
 (segment (start 147.035 87.845) (end 146.735001 87.545001) (width 0.5) (layer "F.Cu") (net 1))
 (segment (start 155.17 88.234925) (end 155.17 84.79) (width 0.5) (layer "F.Cu") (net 7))
 (segment (start 154.289925 89.115) (end 155.17 88.234925) (width 0.5) (layer "F.Cu") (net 7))
 (segment (start 151.985 89.115) (end 154.289925 89.115) (width 0.5) (layer "F.Cu") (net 7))
 (segment (start 155.17 84.79) (end 152.68 82.3) (width 0.5) (layer "F.Cu") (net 7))
 (segment (start 152.68 82.3) (end 150.77 82.3) (width 0.5) (layer "F.Cu") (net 7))
 (segment (start 157.455 90.385) (end 158.8 89.04) (width 0.5) (layer "F.Cu") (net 6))
 (segment (start 151.985 90.385) (end 157.455 90.385) (width 0.5) (layer "F.Cu") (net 6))
 (segment (start 158.725 91.655) (end 158.8 91.58) (width 0.5) (layer "F.Cu") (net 5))
 (segment (start 151.985 91.655) (end 158.725 91.655) (width 0.5) (layer "F.Cu") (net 5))
 (segment (start 148.9 88.405) (end 149 88.505) (width 0.5) (layer "F.Cu") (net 4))
 (segment (start 149.5 91.1) (end 148.945 91.655) (width 0.5) (layer "F.Cu") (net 4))
 (segment (start 149.51 89.75) (end 149.5 89.76) (width 0.5) (layer "F.Cu") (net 4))
 (segment (start 148.945 91.655) (end 147.035 91.655) (width 0.5) (layer "F.Cu") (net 4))
 (segment (start 149.5 89.76) (end 149.5 91.1) (width 0.5) (layer "F.Cu") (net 4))
 (via (at 143.41 90.43) (size 0.8) (drill 0.4) (layers "F.Cu" "B.Cu") (free) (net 4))
 (via (at 157.15 94.7) (size 0.8) (drill 0.4) (layers "F.Cu" "B.Cu") (free) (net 4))
 (via (at 144.66 85.08) (size 0.8) (drill 0.4) (layers "F.Cu" "B.Cu") (free) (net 4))
 (via (at 140.87 81.86) (size 0.8) (drill 0.4) (layers "F.Cu" "B.Cu") (free) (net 4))
 (via (at 150.05 93.15) (size 0.8) (drill 0.4) (layers "F.Cu" "B.Cu") (free) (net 4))
 (via (at 157.63 82.63) (size 0.8) (drill 0.4) (layers "F.Cu" "B.Cu") (free) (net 4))
 (via (at 141.86 94.9) (size 0.8) (drill 0.4) (layers "F.Cu" "B.Cu") (free) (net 4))
 (via (at 149.55 85.88) (size 0.8) (drill 0.4) (layers "F.Cu" "B.Cu") (free) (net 4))
 (segment (start 151.985 87.845) (end 152.355 87.845) (width 0.5) (layer "F.Cu") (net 8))
 (segment (start 152.1 85.87) (end 152.1 87.73) (width 0.8) (layer "F.Cu") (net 8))
 (segment (start 151.985 87.845) (end 152.1 87.73) (width 0.5) (layer "F.Cu") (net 8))
 (via (at 152.1 85.87) (size 1.4) (drill 0.8) (layers "F.Cu" "B.Cu") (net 8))
 (segment (start 152.73 86.5) (end 152.1 85.87) (width 0.8) (layer "B.Cu") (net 8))
 (segment (start 158.8 86.5) (end 152.73 86.5) (width 0.8) (layer "B.Cu") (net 8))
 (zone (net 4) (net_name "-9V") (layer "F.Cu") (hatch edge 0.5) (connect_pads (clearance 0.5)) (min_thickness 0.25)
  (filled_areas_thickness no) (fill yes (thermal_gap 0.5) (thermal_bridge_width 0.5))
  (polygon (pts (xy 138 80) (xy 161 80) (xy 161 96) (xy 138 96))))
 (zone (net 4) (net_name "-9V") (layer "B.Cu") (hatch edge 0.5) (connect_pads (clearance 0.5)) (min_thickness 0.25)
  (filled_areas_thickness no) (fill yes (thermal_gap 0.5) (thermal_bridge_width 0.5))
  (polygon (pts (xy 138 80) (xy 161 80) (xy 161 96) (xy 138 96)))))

